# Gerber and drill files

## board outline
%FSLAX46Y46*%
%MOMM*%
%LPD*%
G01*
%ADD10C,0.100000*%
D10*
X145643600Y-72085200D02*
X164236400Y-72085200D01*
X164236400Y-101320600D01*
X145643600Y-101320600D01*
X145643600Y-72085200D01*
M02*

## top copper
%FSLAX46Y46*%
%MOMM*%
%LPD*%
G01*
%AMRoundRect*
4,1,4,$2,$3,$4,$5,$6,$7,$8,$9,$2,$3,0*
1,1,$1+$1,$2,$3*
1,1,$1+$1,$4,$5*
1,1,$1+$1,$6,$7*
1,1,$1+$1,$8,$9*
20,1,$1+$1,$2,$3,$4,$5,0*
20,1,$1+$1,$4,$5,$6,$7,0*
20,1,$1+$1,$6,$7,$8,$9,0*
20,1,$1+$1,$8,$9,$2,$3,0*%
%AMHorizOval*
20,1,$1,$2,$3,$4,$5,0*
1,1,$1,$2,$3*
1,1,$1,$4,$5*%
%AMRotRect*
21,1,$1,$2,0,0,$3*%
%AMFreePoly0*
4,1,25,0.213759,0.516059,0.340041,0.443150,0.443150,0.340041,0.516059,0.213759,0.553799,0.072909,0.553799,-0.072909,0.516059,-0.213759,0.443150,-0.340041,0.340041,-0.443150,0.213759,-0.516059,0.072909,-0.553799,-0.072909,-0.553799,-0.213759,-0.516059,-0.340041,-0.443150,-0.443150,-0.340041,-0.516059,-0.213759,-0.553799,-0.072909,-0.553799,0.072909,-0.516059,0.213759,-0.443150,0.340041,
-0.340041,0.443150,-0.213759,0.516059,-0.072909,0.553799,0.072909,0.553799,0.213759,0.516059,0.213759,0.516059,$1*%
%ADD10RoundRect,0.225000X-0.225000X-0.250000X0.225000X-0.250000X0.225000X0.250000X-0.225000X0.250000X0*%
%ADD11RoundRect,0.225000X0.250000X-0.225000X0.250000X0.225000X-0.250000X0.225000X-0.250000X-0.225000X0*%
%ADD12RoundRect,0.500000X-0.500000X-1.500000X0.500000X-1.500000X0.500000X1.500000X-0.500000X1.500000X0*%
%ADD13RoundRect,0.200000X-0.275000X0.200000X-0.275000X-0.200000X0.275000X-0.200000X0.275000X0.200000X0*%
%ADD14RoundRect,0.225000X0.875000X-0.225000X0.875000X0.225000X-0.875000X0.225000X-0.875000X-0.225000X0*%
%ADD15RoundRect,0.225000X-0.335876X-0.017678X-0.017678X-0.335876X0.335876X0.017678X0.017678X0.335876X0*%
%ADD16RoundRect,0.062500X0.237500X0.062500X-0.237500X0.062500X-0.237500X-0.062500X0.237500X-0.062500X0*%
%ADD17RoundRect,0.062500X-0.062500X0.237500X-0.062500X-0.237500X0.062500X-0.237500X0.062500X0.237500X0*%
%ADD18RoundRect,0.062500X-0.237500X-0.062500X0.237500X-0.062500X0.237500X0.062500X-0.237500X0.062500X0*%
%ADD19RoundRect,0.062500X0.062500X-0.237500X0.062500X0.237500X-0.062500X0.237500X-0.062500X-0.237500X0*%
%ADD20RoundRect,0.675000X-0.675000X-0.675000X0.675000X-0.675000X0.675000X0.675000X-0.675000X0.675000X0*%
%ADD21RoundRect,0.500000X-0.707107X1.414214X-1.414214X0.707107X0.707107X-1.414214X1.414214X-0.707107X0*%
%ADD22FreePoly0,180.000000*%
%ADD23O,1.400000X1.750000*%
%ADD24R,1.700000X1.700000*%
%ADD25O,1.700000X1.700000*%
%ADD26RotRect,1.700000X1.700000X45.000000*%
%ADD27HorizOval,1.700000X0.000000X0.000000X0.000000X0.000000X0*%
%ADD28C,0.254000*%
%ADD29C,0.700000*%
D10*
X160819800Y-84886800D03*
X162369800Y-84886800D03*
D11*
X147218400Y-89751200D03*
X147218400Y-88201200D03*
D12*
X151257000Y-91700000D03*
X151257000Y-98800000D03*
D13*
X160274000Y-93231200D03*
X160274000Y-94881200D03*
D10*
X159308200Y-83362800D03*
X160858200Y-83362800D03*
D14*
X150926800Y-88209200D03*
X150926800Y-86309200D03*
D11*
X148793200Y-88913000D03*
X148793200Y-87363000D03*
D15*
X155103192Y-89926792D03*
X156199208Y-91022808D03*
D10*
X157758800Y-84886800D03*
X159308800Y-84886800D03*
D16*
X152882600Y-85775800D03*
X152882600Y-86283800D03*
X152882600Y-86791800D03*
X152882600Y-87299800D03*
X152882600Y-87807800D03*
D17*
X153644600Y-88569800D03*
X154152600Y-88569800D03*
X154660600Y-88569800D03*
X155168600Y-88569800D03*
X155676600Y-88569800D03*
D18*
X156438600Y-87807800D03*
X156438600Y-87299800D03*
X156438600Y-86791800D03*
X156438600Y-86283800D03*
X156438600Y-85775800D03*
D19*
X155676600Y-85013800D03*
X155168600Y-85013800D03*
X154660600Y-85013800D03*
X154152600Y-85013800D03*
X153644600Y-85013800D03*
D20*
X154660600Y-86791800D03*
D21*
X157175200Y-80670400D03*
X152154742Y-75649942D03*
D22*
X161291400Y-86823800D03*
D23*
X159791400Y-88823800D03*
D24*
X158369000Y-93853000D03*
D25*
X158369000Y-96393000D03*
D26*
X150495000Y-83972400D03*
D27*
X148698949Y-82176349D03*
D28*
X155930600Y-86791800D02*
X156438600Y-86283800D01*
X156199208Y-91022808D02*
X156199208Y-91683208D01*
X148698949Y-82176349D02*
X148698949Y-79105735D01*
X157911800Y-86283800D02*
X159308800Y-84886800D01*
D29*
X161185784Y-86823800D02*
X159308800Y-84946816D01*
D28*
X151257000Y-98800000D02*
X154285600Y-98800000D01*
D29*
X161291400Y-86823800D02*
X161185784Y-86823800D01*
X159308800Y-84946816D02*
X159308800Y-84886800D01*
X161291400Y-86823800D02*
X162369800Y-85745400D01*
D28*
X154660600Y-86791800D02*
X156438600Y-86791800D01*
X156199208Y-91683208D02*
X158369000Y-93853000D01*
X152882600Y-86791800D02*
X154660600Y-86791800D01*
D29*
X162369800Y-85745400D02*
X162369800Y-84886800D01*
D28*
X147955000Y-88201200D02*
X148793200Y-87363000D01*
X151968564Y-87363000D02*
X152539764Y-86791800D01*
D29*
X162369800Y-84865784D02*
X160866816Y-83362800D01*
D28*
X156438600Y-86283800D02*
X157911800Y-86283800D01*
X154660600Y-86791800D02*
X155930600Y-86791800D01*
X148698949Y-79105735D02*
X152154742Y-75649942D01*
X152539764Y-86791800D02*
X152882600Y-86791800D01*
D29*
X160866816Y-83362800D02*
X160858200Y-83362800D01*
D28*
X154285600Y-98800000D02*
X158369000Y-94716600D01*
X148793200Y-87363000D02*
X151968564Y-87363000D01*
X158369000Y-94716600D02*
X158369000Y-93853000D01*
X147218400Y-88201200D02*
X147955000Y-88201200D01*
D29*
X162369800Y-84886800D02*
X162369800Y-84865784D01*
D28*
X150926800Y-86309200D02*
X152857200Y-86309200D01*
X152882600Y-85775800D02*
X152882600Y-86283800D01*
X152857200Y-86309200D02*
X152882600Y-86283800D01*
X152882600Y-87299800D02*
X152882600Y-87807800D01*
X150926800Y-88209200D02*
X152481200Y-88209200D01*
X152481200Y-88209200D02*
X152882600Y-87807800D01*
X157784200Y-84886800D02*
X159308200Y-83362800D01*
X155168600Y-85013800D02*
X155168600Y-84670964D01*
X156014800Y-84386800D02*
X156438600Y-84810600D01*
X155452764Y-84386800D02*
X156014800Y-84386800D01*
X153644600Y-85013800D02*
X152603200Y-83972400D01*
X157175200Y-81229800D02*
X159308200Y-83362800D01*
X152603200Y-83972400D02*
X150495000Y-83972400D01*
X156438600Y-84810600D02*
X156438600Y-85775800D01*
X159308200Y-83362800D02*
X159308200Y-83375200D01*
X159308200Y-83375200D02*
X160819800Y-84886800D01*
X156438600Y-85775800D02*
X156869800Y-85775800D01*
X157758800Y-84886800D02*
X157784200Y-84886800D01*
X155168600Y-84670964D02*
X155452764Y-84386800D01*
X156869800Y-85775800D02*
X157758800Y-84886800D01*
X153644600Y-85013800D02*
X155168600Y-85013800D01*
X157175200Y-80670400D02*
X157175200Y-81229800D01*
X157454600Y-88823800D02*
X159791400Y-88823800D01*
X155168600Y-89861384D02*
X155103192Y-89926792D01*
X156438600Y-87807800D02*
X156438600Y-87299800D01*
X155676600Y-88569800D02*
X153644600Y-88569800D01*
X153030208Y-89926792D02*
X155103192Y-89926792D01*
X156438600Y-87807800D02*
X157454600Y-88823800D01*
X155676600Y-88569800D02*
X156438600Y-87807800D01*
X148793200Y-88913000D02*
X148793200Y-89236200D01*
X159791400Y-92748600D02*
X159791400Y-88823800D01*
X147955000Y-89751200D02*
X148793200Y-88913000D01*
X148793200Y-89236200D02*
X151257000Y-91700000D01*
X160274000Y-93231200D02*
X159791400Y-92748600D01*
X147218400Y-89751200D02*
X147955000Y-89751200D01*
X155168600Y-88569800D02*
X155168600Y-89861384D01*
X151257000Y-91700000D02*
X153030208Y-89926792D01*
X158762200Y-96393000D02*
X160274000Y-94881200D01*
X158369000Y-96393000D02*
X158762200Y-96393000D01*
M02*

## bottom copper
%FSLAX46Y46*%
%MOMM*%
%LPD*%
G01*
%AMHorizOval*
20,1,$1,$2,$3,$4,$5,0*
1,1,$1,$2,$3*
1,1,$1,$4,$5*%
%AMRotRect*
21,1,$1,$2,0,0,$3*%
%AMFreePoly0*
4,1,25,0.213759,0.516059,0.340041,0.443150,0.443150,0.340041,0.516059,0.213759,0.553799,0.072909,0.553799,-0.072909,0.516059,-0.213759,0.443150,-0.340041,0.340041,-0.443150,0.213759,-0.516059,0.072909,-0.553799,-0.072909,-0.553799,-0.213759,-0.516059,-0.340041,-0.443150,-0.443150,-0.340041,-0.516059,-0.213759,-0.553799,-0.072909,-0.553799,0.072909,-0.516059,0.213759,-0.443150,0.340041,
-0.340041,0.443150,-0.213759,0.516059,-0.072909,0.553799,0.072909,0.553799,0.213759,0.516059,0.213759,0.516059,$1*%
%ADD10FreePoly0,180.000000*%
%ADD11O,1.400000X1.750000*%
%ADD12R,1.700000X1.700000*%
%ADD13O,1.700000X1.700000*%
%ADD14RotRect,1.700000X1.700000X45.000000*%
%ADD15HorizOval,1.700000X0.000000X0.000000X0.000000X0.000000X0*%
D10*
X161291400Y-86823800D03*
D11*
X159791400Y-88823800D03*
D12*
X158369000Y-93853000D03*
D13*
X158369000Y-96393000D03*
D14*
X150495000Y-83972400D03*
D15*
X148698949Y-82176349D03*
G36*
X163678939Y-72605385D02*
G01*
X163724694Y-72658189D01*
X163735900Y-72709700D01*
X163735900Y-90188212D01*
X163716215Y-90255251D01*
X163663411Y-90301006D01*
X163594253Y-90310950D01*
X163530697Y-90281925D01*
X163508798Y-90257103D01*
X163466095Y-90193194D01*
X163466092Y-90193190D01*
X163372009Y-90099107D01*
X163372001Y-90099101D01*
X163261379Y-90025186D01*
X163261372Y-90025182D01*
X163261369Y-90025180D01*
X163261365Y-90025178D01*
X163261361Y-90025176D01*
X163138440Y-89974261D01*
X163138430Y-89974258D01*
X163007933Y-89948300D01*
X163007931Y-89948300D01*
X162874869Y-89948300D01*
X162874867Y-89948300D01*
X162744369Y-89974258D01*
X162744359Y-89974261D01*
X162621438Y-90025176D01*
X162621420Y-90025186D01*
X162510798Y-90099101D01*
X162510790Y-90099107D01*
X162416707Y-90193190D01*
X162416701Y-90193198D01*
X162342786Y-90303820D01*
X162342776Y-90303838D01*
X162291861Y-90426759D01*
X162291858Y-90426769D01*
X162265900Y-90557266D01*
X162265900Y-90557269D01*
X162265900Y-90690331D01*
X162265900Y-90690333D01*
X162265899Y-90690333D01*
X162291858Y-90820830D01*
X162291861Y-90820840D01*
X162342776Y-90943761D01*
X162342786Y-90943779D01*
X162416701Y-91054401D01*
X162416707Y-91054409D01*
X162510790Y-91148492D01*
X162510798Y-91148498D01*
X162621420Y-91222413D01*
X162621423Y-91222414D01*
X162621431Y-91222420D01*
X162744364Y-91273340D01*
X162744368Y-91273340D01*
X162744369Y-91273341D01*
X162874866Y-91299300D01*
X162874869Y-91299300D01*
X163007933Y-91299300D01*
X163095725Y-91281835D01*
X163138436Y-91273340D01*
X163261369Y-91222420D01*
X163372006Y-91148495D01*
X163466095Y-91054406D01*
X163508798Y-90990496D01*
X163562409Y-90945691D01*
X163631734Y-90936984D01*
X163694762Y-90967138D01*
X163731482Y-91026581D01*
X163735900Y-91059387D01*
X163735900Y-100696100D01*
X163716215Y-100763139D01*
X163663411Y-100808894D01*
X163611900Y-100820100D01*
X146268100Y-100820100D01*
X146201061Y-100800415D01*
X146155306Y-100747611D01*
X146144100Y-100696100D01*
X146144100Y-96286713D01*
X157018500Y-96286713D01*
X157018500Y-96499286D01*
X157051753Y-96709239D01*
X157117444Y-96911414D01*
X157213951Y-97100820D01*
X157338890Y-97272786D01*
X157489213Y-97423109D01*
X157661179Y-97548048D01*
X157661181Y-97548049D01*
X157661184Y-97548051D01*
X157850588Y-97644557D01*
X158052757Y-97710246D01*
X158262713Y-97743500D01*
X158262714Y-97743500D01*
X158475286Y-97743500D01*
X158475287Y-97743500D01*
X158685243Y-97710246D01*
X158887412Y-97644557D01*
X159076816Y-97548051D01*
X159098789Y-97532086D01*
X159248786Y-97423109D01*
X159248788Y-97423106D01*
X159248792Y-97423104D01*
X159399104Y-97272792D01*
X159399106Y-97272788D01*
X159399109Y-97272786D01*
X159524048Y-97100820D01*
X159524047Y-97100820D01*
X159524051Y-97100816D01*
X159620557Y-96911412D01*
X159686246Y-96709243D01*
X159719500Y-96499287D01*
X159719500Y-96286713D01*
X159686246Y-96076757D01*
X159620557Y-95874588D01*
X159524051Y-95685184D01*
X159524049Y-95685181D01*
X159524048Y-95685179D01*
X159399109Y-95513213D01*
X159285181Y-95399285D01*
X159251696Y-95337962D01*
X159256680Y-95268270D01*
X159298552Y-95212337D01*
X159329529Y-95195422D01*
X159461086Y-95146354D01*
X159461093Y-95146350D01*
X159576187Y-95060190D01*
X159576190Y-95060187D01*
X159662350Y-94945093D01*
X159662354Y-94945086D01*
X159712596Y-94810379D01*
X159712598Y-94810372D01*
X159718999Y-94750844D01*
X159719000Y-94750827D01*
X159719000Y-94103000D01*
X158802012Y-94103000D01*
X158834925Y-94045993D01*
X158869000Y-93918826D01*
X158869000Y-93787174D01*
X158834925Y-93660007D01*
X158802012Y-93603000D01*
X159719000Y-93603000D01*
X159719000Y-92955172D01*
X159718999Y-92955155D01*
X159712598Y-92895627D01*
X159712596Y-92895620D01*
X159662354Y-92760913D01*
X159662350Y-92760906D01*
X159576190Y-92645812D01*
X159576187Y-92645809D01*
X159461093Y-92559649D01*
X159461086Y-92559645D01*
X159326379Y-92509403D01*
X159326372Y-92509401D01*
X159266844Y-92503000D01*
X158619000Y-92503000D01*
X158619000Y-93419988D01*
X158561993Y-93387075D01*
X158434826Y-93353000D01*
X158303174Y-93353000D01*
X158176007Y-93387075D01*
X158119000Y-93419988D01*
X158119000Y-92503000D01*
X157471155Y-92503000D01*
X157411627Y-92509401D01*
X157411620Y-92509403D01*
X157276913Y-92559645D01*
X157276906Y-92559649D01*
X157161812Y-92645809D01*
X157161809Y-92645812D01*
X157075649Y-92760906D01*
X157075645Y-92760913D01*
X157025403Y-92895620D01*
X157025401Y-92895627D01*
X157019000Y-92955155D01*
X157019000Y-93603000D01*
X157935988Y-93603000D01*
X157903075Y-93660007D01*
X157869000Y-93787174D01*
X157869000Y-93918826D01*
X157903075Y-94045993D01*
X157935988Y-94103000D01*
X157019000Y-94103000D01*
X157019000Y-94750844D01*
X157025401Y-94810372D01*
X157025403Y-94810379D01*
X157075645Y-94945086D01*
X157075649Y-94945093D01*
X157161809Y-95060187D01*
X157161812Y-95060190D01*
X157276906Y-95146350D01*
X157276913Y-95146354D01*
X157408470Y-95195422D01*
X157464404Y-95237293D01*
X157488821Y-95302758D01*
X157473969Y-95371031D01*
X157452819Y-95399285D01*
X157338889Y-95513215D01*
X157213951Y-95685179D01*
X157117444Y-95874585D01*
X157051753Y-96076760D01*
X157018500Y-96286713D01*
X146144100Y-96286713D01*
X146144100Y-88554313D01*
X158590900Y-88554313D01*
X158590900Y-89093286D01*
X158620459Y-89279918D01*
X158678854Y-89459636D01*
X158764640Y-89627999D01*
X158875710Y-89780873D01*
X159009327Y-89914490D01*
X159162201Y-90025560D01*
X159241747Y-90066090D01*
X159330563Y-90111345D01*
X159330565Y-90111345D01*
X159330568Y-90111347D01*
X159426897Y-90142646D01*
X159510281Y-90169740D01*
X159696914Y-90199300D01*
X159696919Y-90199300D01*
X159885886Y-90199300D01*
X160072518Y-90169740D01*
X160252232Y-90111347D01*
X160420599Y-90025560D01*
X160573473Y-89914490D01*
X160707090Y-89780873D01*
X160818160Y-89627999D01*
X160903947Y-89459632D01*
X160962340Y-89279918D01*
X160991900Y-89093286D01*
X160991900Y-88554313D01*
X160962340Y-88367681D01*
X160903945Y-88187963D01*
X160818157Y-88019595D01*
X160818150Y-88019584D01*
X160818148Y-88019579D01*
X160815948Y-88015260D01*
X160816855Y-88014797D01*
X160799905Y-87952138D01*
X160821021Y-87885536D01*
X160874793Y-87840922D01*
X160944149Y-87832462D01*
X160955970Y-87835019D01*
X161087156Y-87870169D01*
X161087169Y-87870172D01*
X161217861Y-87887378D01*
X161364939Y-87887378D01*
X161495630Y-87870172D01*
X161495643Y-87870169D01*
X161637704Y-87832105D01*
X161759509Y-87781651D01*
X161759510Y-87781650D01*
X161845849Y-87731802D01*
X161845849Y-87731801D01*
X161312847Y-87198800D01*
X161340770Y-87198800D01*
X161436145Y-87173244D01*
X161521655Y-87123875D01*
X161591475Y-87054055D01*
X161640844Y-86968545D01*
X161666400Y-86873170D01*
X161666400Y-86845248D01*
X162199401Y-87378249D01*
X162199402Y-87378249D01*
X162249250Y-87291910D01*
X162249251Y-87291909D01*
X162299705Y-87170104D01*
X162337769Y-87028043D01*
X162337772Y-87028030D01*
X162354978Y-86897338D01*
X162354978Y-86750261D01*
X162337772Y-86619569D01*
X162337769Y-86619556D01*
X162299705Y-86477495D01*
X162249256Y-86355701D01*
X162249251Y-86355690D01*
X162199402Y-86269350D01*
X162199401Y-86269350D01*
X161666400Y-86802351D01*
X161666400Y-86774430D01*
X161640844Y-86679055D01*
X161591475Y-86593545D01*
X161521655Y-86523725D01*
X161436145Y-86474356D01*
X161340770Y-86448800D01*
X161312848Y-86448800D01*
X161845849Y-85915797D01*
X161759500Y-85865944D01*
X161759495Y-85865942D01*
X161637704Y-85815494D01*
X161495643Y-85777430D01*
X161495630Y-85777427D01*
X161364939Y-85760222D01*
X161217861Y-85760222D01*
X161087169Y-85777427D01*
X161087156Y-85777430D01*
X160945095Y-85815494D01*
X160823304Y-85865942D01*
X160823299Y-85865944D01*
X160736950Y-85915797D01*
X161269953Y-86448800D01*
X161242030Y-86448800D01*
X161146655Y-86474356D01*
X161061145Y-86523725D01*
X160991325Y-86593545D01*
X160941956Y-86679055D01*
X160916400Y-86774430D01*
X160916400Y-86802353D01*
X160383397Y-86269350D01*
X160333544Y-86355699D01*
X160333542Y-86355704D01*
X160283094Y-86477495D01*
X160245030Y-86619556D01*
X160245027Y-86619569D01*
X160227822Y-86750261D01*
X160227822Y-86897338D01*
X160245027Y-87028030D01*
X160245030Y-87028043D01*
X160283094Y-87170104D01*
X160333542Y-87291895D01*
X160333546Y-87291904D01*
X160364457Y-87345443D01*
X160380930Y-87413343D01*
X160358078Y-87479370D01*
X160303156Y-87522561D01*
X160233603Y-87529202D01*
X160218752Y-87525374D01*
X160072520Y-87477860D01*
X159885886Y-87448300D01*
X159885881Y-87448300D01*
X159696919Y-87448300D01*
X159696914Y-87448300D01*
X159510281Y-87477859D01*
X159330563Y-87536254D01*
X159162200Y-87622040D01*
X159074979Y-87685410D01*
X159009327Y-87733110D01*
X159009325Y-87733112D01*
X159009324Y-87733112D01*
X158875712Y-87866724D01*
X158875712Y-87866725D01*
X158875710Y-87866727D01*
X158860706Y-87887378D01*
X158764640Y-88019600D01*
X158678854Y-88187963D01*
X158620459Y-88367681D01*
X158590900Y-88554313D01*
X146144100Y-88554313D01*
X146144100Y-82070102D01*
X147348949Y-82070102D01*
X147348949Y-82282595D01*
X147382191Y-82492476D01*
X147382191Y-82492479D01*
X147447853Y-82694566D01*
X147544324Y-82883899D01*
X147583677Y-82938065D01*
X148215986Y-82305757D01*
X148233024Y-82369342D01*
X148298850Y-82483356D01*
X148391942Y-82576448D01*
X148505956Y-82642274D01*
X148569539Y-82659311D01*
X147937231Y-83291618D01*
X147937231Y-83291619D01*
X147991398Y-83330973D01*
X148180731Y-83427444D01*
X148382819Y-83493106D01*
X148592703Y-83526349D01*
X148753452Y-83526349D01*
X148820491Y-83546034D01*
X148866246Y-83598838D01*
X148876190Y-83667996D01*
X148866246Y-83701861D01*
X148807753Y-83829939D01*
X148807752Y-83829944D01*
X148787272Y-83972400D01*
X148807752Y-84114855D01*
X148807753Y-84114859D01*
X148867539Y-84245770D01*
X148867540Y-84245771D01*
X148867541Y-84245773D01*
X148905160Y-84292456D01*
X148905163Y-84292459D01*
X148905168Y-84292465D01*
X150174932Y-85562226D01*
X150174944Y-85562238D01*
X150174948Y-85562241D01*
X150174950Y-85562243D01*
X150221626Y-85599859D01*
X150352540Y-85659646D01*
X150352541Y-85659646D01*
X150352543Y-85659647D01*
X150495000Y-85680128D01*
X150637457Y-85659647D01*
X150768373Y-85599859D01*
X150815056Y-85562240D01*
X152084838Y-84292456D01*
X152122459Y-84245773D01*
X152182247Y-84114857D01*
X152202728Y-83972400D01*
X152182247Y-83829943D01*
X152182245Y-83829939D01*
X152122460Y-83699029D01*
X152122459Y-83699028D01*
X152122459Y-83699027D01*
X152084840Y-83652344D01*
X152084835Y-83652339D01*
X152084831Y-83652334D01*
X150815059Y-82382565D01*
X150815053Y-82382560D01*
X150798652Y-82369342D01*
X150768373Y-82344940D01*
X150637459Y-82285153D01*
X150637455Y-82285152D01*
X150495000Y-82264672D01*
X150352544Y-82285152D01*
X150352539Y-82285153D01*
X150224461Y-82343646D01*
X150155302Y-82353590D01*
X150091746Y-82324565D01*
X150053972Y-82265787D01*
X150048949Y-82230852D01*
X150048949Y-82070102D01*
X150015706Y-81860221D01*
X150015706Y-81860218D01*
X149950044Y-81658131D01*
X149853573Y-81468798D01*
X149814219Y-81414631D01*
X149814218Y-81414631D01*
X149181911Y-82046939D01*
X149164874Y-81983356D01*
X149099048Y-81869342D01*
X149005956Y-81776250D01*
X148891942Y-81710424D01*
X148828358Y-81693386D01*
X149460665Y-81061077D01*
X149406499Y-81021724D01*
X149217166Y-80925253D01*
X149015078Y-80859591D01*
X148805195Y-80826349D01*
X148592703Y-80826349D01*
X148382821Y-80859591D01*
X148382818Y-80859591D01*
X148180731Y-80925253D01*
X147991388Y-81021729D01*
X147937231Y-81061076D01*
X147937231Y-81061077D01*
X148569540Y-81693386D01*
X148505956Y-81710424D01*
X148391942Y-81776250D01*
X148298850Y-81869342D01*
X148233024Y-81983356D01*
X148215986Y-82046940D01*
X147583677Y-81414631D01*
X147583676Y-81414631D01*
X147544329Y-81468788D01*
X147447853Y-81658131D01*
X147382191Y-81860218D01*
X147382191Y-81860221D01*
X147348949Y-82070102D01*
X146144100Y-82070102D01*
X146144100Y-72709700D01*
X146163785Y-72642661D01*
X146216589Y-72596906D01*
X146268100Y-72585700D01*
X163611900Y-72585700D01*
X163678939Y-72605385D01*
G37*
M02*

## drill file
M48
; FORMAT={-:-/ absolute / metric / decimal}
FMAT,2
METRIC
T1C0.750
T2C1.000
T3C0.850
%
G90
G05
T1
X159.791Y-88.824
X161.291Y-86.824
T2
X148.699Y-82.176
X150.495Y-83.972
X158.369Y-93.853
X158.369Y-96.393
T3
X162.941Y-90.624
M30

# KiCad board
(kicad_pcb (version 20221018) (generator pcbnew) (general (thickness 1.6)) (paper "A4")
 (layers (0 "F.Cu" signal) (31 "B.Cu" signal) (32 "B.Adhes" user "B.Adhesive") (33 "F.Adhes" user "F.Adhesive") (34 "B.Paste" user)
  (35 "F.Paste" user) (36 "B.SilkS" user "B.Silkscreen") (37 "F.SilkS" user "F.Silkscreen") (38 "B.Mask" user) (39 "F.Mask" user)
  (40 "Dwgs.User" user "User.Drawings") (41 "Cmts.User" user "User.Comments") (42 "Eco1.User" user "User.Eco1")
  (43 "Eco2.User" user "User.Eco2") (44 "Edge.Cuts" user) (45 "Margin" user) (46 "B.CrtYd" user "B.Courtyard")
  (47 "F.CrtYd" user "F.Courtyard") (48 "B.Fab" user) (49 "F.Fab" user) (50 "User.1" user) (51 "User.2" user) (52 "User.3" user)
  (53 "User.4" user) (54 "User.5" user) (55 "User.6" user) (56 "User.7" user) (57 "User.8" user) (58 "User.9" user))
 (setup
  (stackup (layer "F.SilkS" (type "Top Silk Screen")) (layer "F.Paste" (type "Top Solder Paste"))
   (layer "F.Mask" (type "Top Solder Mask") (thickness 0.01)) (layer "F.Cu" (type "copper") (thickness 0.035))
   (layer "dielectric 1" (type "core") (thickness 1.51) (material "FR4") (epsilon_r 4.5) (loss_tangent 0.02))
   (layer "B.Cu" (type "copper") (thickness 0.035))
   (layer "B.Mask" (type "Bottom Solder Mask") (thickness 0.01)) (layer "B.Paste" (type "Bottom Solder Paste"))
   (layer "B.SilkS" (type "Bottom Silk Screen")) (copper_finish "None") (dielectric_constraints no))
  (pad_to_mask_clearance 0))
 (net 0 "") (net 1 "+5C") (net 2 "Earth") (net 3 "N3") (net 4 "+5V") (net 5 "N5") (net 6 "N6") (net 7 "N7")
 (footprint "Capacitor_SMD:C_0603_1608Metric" (layer "F.Cu") (at 161.5948 84.8868)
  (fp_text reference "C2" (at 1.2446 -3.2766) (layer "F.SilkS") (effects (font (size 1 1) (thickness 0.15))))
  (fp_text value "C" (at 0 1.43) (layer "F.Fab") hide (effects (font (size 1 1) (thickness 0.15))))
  (pad "1" smd roundrect (at -0.775 0) (size 0.9 0.95) (layers "F.Cu" "F.Paste" "F.Mask") (roundrect_rratio 0.25) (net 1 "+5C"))
  (pad "2" smd roundrect (at 0.775 0) (size 0.9 0.95) (layers "F.Cu" "F.Paste" "F.Mask") (roundrect_rratio 0.25) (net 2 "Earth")))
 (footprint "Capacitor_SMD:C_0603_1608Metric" (layer "F.Cu") (at 147.2184 88.9762 90)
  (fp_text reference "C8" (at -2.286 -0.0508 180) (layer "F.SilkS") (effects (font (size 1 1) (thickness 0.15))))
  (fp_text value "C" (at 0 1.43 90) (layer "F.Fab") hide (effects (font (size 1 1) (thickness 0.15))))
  (pad "1" smd roundrect (at -0.775 0 90) (size 0.9 0.95) (layers "F.Cu" "F.Paste" "F.Mask") (roundrect_rratio 0.25) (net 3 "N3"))
  (pad "2" smd roundrect (at 0.775 0 90) (size 0.9 0.95) (layers "F.Cu" "F.Paste" "F.Mask") (roundrect_rratio 0.25) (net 2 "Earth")))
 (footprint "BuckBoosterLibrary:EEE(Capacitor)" (layer "F.Cu") (at 151.257 95.25)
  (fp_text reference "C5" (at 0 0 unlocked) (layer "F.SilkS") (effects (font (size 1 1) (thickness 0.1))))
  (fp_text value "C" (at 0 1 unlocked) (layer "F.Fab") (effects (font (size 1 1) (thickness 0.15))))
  (pad "1" smd roundrect (at 0 -3.55) (size 2 4) (layers "F.Cu" "F.Paste" "F.Mask") (roundrect_rratio 0.25) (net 3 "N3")
   (thermal_bridge_angle 45))
  (pad "2" smd roundrect (at 0 3.55) (size 2 4) (layers "F.Cu" "F.Paste" "F.Mask") (roundrect_rratio 0.25) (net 2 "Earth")
   (thermal_bridge_angle 45)))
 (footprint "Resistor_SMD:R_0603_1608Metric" (layer "F.Cu") (at 160.274 94.0562 -90)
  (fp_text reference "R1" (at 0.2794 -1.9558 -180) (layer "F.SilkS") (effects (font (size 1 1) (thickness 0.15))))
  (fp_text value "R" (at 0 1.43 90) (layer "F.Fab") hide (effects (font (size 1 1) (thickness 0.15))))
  (pad "1" smd roundrect (at -0.825 0 270) (size 0.8 0.95) (layers "F.Cu" "F.Paste" "F.Mask") (roundrect_rratio 0.25) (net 3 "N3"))
  (pad "2" smd roundrect (at 0.825 0 270) (size 0.8 0.95) (layers "F.Cu" "F.Paste" "F.Mask") (roundrect_rratio 0.25) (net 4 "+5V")))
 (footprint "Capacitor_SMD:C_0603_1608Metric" (layer "F.Cu") (at 160.0832 83.3628)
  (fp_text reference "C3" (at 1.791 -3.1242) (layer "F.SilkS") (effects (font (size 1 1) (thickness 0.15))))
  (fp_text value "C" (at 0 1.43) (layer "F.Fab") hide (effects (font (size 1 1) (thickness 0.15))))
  (pad "1" smd roundrect (at -0.775 0) (size 0.9 0.95) (layers "F.Cu" "F.Paste" "F.Mask") (roundrect_rratio 0.25) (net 1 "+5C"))
  (pad "2" smd roundrect (at 0.775 0) (size 0.9 0.95) (layers "F.Cu" "F.Paste" "F.Mask") (roundrect_rratio 0.25) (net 2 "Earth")))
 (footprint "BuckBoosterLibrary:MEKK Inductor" (layer "F.Cu") (at 150.9268 87.2592 90)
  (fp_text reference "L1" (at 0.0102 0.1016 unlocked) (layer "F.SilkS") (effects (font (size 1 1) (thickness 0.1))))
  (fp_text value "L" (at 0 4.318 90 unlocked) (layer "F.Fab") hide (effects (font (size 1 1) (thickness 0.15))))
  (pad "1" smd roundrect (at -0.95 0 90) (size 0.9 2.2) (layers "F.Cu" "F.Paste" "F.Mask") (roundrect_rratio 0.25) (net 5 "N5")
   (thermal_bridge_angle 45))
  (pad "2" smd roundrect (at 0.95 0 90) (size 0.9 2.2) (layers "F.Cu" "F.Paste" "F.Mask") (roundrect_rratio 0.25) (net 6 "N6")
   (thermal_bridge_angle 45)))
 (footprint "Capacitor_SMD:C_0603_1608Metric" (layer "F.Cu") (at 148.7932 88.138 90)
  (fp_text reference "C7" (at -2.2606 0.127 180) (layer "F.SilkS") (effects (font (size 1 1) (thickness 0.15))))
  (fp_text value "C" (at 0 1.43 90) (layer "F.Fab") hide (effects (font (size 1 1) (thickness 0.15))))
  (pad "1" smd roundrect (at -0.775 0 90) (size 0.9 0.95) (layers "F.Cu" "F.Paste" "F.Mask") (roundrect_rratio 0.25) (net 3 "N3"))
  (pad "2" smd roundrect (at 0.775 0 90) (size 0.9 0.95) (layers "F.Cu" "F.Paste" "F.Mask") (roundrect_rratio 0.25) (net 2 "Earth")))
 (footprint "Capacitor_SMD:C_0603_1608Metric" (layer "F.Cu") (at 155.6512 90.4748 -45)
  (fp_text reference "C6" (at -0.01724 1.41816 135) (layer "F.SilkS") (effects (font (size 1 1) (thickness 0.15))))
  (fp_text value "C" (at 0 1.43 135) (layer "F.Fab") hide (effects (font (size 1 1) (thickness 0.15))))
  (pad "1" smd roundrect (at -0.775 0 315) (size 0.9 0.95) (layers "F.Cu" "F.Paste" "F.Mask") (roundrect_rratio 0.25) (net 3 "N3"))
  (pad "2" smd roundrect (at 0.775 0 315) (size 0.9 0.95) (layers "F.Cu" "F.Paste" "F.Mask") (roundrect_rratio 0.25) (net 2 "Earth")))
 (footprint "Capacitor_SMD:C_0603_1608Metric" (layer "F.Cu") (at 158.5338 84.8868)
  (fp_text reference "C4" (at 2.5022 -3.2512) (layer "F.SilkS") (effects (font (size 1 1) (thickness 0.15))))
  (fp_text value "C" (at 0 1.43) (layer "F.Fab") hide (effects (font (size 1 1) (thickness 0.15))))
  (pad "1" smd roundrect (at -0.775 0) (size 0.9 0.95) (layers "F.Cu" "F.Paste" "F.Mask") (roundrect_rratio 0.25) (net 1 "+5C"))
  (pad "2" smd roundrect (at 0.775 0) (size 0.9 0.95) (layers "F.Cu" "F.Paste" "F.Mask") (roundrect_rratio 0.25) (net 2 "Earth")))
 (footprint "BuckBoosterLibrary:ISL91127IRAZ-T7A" (layer "F.Cu") (at 154.6606 86.7918)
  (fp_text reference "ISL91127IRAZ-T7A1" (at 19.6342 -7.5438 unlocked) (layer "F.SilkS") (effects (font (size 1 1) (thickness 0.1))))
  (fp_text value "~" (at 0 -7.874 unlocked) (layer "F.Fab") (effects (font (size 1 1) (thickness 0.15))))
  (pad "1" smd roundrect (at -1.778 -1.016 180) (size 0.6 0.25) (layers "F.Cu" "F.Paste" "F.Mask") (roundrect_rratio 0.25) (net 6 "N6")
   (thermal_bridge_angle 45))
  (pad "2" smd roundrect (at -1.778 -0.508 180) (size 0.6 0.25) (layers "F.Cu" "F.Paste" "F.Mask") (roundrect_rratio 0.25) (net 6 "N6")
   (thermal_bridge_angle 45))
  (pad "3" smd roundrect (at -1.778 0 180) (size 0.6 0.25) (layers "F.Cu" "F.Paste" "F.Mask") (roundrect_rratio 0.25) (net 2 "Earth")
   (thermal_bridge_angle 45))
  (pad "4" smd roundrect (at -1.778 0.508 180) (size 0.6 0.25) (layers "F.Cu" "F.Paste" "F.Mask") (roundrect_rratio 0.25) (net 5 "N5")
   (thermal_bridge_angle 45))
  (pad "5" smd roundrect (at -1.778 1.016 180) (size 0.6 0.25) (layers "F.Cu" "F.Paste" "F.Mask") (roundrect_rratio 0.25) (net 5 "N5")
   (thermal_bridge_angle 45))
  (pad "6" smd roundrect (at -1.016 1.778 270) (size 0.6 0.25) (layers "F.Cu" "F.Paste" "F.Mask") (roundrect_rratio 0.25) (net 3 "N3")
   (thermal_bridge_angle 45))
  (pad "7" smd roundrect (at -0.508 1.778 270) (size 0.6 0.25) (layers "F.Cu" "F.Paste" "F.Mask") (roundrect_rratio 0.25) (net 3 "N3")
   (thermal_bridge_angle 45))
  (pad "8" smd roundrect (at 0 1.778 270) (size 0.6 0.25) (layers "F.Cu" "F.Paste" "F.Mask") (roundrect_rratio 0.25) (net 3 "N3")
   (thermal_bridge_angle 45))
  (pad "9" smd roundrect (at 0.508 1.778 270) (size 0.6 0.25) (layers "F.Cu" "F.Paste" "F.Mask") (roundrect_rratio 0.25) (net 3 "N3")
   (thermal_bridge_angle 45))
  (pad "10" smd roundrect (at 1.016 1.778 270) (size 0.6 0.25) (layers "F.Cu" "F.Paste" "F.Mask") (roundrect_rratio 0.25) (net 3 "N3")
   (thermal_bridge_angle 45))
  (pad "11" smd roundrect (at 1.778 1.016) (size 0.6 0.25) (layers "F.Cu" "F.Paste" "F.Mask") (roundrect_rratio 0.25) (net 3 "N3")
   (thermal_bridge_angle 45))
  (pad "12" smd roundrect (at 1.778 0.508) (size 0.6 0.25) (layers "F.Cu" "F.Paste" "F.Mask") (roundrect_rratio 0.25) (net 3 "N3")
   (thermal_bridge_angle 45))
  (pad "13" smd roundrect (at 1.778 0) (size 0.6 0.25) (layers "F.Cu" "F.Paste" "F.Mask") (roundrect_rratio 0.25) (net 2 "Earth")
   (thermal_bridge_angle 45))
  (pad "14" smd roundrect (at 1.778 -0.508) (size 0.6 0.25) (layers "F.Cu" "F.Paste" "F.Mask") (roundrect_rratio 0.25) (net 2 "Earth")
   (thermal_bridge_angle 45))
  (pad "15" smd roundrect (at 1.778 -1.016) (size 0.6 0.25) (layers "F.Cu" "F.Paste" "F.Mask") (roundrect_rratio 0.25) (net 1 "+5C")
   (thermal_bridge_angle 45))
  (pad "16" smd roundrect (at 1.016 -1.778 90) (size 0.6 0.25) (layers "F.Cu" "F.Paste" "F.Mask") (roundrect_rratio 0.25) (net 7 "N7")
   (thermal_bridge_angle 45))
  (pad "17" smd roundrect (at 0.508 -1.778 90) (size 0.6 0.25) (layers "F.Cu" "F.Paste" "F.Mask") (roundrect_rratio 0.25) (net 1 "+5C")
   (thermal_bridge_angle 45))
  (pad "18" smd roundrect (at 0 -1.778 90) (size 0.6 0.25) (layers "F.Cu" "F.Paste" "F.Mask") (roundrect_rratio 0.25) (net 1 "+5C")
   (thermal_bridge_angle 45))
  (pad "19" smd roundrect (at -0.508 -1.778 90) (size 0.6 0.25) (layers "F.Cu" "F.Paste" "F.Mask") (roundrect_rratio 0.25) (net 1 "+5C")
   (thermal_bridge_angle 45))
  (pad "20" smd roundrect (at -1.016 -1.778 90) (size 0.6 0.25) (layers "F.Cu" "F.Paste" "F.Mask") (roundrect_rratio 0.25) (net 1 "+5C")
   (thermal_bridge_angle 45))
  (pad "21" smd roundrect (at 0 0) (size 2.7 2.7) (layers "F.Cu" "F.Paste" "F.Mask") (roundrect_rratio 0.25) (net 2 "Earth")
   (thermal_bridge_angle 45)))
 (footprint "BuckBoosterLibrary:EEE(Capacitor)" (layer "F.Cu") (at 154.664971 78.160171 -135)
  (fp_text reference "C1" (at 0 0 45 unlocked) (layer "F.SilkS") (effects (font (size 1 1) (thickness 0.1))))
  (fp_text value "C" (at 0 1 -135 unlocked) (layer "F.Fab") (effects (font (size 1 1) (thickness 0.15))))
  (pad "1" smd roundrect (at 0 -3.55 225) (size 2 4) (layers "F.Cu" "F.Paste" "F.Mask") (roundrect_rratio 0.25) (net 1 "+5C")
   (thermal_bridge_angle 45))
  (pad "2" smd roundrect (at 0 3.55 225) (size 2 4) (layers "F.Cu" "F.Paste" "F.Mask") (roundrect_rratio 0.25) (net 2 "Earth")
   (thermal_bridge_angle 45)))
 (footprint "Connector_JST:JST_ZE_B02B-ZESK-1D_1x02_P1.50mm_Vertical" (layer "F.Cu") (at 161.2914 86.8238 180)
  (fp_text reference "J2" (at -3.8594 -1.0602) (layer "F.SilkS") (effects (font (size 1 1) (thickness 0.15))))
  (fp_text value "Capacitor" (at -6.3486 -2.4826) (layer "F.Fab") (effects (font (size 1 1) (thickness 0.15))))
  (pad "" np_thru_hole circle (at -1.65 -3.8 180) (size 0.85 0.85) (drill 0.85) (layers "*.Cu" "*.Mask"))
  (pad "1" thru_hole custom (at 0 0 180) (size 1.117157 1.117157) (drill 0.75) (layers "*.Cu" "*.Mask") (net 2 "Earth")
   (thermal_bridge_angle 45) (options (clearance outline) (anchor circle)) (primitives))
  (pad "2" thru_hole oval (at 1.5 -2 180) (size 1.4 1.75) (drill 0.75) (layers "*.Cu" "*.Mask") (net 3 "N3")))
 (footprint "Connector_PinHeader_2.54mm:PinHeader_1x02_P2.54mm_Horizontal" (layer "B.Cu") (at 158.369 93.853 180)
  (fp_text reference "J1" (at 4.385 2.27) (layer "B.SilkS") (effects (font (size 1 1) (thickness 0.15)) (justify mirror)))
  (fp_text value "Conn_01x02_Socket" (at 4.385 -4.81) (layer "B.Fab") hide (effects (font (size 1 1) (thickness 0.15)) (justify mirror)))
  (pad "1" thru_hole rect (at 0 0 180) (size 1.7 1.7) (drill 1) (layers "*.Cu" "*.Mask") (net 2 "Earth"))
  (pad "2" thru_hole oval (at 0 -2.54 180) (size 1.7 1.7) (drill 1) (layers "*.Cu" "*.Mask") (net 4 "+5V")))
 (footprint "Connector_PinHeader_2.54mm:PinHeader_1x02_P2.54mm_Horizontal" (layer "B.Cu") (at 150.495 83.9724 45)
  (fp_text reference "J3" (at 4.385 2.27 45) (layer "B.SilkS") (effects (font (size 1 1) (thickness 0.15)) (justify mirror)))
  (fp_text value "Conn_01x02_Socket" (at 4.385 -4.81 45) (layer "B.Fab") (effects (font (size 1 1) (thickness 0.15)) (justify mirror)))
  (pad "1" thru_hole rect (at 0 0 45) (size 1.7 1.7) (drill 1) (layers "*.Cu" "*.Mask") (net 1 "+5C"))
  (pad "2" thru_hole oval (at 0 -2.54 45) (size 1.7 1.7) (drill 1) (layers "*.Cu" "*.Mask") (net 2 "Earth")))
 (gr_rect (start 145.6436 72.0852) (end 164.2364 101.3206) (stroke (width 0.1) (type default)) (fill none) (layer "Edge.Cuts"))
 (segment (start 155.9306 86.7918) (end 156.4386 86.2838) (width 0.254) (layer "F.Cu") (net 2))
 (segment (start 156.199208 91.022808) (end 156.199208 91.683208) (width 0.254) (layer "F.Cu") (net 2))
 (segment (start 148.698949 82.176349) (end 148.698949 79.105735) (width 0.254) (layer "F.Cu") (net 2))
 (segment (start 157.9118 86.2838) (end 159.3088 84.8868) (width 0.254) (layer "F.Cu") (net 2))
 (segment (start 161.185784 86.8238) (end 159.3088 84.946816) (width 0.7) (layer "F.Cu") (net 2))
 (segment (start 151.257 98.8) (end 154.2856 98.8) (width 0.254) (layer "F.Cu") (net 2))
 (segment (start 161.2914 86.8238) (end 161.185784 86.8238) (width 0.7) (layer "F.Cu") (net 2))
 (segment (start 159.3088 84.946816) (end 159.3088 84.8868) (width 0.7) (layer "F.Cu") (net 2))
 (segment (start 161.2914 86.8238) (end 162.3698 85.7454) (width 0.7) (layer "F.Cu") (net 2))
 (segment (start 154.6606 86.7918) (end 156.4386 86.7918) (width 0.254) (layer "F.Cu") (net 2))
 (segment (start 156.199208 91.683208) (end 158.369 93.853) (width 0.254) (layer "F.Cu") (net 2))
 (segment (start 152.8826 86.7918) (end 154.6606 86.7918) (width 0.254) (layer "F.Cu") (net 2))
 (segment (start 162.3698 85.7454) (end 162.3698 84.8868) (width 0.7) (layer "F.Cu") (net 2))
 (segment (start 147.955 88.2012) (end 148.7932 87.363) (width 0.254) (layer "F.Cu") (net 2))
 (segment (start 151.968564 87.363) (end 152.539764 86.7918) (width 0.254) (layer "F.Cu") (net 2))
 (segment (start 162.3698 84.865784) (end 160.866816 83.3628) (width 0.7) (layer "F.Cu") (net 2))
 (segment (start 156.4386 86.2838) (end 157.9118 86.2838) (width 0.254) (layer "F.Cu") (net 2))
 (segment (start 154.6606 86.7918) (end 155.9306 86.7918) (width 0.254) (layer "F.Cu") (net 2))
 (segment (start 148.698949 79.105735) (end 152.154742 75.649942) (width 0.254) (layer "F.Cu") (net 2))
 (segment (start 152.539764 86.7918) (end 152.8826 86.7918) (width 0.254) (layer "F.Cu") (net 2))
 (segment (start 160.866816 83.3628) (end 160.8582 83.3628) (width 0.7) (layer "F.Cu") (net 2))
 (segment (start 154.2856 98.8) (end 158.369 94.7166) (width 0.254) (layer "F.Cu") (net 2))
 (segment (start 148.7932 87.363) (end 151.968564 87.363) (width 0.254) (layer "F.Cu") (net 2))
 (segment (start 158.369 94.7166) (end 158.369 93.853) (width 0.254) (layer "F.Cu") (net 2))
 (segment (start 147.2184 88.2012) (end 147.955 88.2012) (width 0.254) (layer "F.Cu") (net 2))
 (segment (start 162.3698 84.8868) (end 162.3698 84.865784) (width 0.7) (layer "F.Cu") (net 2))
 (segment (start 150.9268 86.3092) (end 152.8572 86.3092) (width 0.254) (layer "F.Cu") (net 6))
 (segment (start 152.8826 85.7758) (end 152.8826 86.2838) (width 0.254) (layer "F.Cu") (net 6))
 (segment (start 152.8572 86.3092) (end 152.8826 86.2838) (width 0.254) (layer "F.Cu") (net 6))
 (segment (start 152.8826 87.2998) (end 152.8826 87.8078) (width 0.254) (layer "F.Cu") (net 5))
 (segment (start 150.9268 88.2092) (end 152.4812 88.2092) (width 0.254) (layer "F.Cu") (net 5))
 (segment (start 152.4812 88.2092) (end 152.8826 87.8078) (width 0.254) (layer "F.Cu") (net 5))
 (segment (start 157.7842 84.8868) (end 159.3082 83.3628) (width 0.254) (layer "F.Cu") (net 1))
 (segment (start 155.1686 85.0138) (end 155.1686 84.670964) (width 0.254) (layer "F.Cu") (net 1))
 (segment (start 156.0148 84.3868) (end 156.4386 84.8106) (width 0.254) (layer "F.Cu") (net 1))
 (segment (start 155.452764 84.3868) (end 156.0148 84.3868) (width 0.254) (layer "F.Cu") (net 1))
 (segment (start 153.6446 85.0138) (end 152.6032 83.9724) (width 0.254) (layer "F.Cu") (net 1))
 (segment (start 157.1752 81.2298) (end 159.3082 83.3628) (width 0.254) (layer "F.Cu") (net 1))
 (segment (start 152.6032 83.9724) (end 150.495 83.9724) (width 0.254) (layer "F.Cu") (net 1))
 (segment (start 156.4386 84.8106) (end 156.4386 85.7758) (width 0.254) (layer "F.Cu") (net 1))
 (segment (start 159.3082 83.3628) (end 159.3082 83.3752) (width 0.254) (layer "F.Cu") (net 1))
 (segment (start 159.3082 83.3752) (end 160.8198 84.8868) (width 0.254) (layer "F.Cu") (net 1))
 (segment (start 156.4386 85.7758) (end 156.8698 85.7758) (width 0.254) (layer "F.Cu") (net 1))
 (segment (start 157.7588 84.8868) (end 157.7842 84.8868) (width 0.254) (layer "F.Cu") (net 1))
 (segment (start 155.1686 84.670964) (end 155.452764 84.3868) (width 0.254) (layer "F.Cu") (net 1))
 (segment (start 156.8698 85.7758) (end 157.7588 84.8868) (width 0.254) (layer "F.Cu") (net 1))
 (segment (start 153.6446 85.0138) (end 155.1686 85.0138) (width 0.254) (layer "F.Cu") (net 1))
 (segment (start 157.1752 80.6704) (end 157.1752 81.2298) (width 0.254) (layer "F.Cu") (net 1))
 (segment (start 157.4546 88.8238) (end 159.7914 88.8238) (width 0.254) (layer "F.Cu") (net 3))
 (segment (start 155.1686 89.861384) (end 155.103192 89.926792) (width 0.254) (layer "F.Cu") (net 3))
 (segment (start 156.4386 87.8078) (end 156.4386 87.2998) (width 0.254) (layer "F.Cu") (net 3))
 (segment (start 155.6766 88.5698) (end 153.6446 88.5698) (width 0.254) (layer "F.Cu") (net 3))
 (segment (start 153.030208 89.926792) (end 155.103192 89.926792) (width 0.254) (layer "F.Cu") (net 3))
 (segment (start 156.4386 87.8078) (end 157.4546 88.8238) (width 0.254) (layer "F.Cu") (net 3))
 (segment (start 155.6766 88.5698) (end 156.4386 87.8078) (width 0.254) (layer "F.Cu") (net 3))
 (segment (start 148.7932 88.913) (end 148.7932 89.2362) (width 0.254) (layer "F.Cu") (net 3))
 (segment (start 159.7914 92.7486) (end 159.7914 88.8238) (width 0.254) (layer "F.Cu") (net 3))
 (segment (start 147.955 89.7512) (end 148.7932 88.913) (width 0.254) (layer "F.Cu") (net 3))
 (segment (start 148.7932 89.2362) (end 151.257 91.7) (width 0.254) (layer "F.Cu") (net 3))
 (segment (start 160.274 93.2312) (end 159.7914 92.7486) (width 0.254) (layer "F.Cu") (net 3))
 (segment (start 147.2184 89.7512) (end 147.955 89.7512) (width 0.254) (layer "F.Cu") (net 3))
 (segment (start 155.1686 88.5698) (end 155.1686 89.861384) (width 0.254) (layer "F.Cu") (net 3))
 (segment (start 151.257 91.7) (end 153.030208 89.926792) (width 0.254) (layer "F.Cu") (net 3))
 (segment (start 158.7622 96.393) (end 160.274 94.8812) (width 0.254) (layer "F.Cu") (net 4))
 (segment (start 158.369 96.393) (end 158.7622 96.393) (width 0.254) (layer "F.Cu") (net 4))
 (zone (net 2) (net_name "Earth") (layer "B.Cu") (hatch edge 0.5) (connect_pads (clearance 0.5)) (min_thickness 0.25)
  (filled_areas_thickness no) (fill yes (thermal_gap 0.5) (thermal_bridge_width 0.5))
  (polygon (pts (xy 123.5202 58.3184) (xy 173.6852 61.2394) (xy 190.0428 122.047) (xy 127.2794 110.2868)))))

